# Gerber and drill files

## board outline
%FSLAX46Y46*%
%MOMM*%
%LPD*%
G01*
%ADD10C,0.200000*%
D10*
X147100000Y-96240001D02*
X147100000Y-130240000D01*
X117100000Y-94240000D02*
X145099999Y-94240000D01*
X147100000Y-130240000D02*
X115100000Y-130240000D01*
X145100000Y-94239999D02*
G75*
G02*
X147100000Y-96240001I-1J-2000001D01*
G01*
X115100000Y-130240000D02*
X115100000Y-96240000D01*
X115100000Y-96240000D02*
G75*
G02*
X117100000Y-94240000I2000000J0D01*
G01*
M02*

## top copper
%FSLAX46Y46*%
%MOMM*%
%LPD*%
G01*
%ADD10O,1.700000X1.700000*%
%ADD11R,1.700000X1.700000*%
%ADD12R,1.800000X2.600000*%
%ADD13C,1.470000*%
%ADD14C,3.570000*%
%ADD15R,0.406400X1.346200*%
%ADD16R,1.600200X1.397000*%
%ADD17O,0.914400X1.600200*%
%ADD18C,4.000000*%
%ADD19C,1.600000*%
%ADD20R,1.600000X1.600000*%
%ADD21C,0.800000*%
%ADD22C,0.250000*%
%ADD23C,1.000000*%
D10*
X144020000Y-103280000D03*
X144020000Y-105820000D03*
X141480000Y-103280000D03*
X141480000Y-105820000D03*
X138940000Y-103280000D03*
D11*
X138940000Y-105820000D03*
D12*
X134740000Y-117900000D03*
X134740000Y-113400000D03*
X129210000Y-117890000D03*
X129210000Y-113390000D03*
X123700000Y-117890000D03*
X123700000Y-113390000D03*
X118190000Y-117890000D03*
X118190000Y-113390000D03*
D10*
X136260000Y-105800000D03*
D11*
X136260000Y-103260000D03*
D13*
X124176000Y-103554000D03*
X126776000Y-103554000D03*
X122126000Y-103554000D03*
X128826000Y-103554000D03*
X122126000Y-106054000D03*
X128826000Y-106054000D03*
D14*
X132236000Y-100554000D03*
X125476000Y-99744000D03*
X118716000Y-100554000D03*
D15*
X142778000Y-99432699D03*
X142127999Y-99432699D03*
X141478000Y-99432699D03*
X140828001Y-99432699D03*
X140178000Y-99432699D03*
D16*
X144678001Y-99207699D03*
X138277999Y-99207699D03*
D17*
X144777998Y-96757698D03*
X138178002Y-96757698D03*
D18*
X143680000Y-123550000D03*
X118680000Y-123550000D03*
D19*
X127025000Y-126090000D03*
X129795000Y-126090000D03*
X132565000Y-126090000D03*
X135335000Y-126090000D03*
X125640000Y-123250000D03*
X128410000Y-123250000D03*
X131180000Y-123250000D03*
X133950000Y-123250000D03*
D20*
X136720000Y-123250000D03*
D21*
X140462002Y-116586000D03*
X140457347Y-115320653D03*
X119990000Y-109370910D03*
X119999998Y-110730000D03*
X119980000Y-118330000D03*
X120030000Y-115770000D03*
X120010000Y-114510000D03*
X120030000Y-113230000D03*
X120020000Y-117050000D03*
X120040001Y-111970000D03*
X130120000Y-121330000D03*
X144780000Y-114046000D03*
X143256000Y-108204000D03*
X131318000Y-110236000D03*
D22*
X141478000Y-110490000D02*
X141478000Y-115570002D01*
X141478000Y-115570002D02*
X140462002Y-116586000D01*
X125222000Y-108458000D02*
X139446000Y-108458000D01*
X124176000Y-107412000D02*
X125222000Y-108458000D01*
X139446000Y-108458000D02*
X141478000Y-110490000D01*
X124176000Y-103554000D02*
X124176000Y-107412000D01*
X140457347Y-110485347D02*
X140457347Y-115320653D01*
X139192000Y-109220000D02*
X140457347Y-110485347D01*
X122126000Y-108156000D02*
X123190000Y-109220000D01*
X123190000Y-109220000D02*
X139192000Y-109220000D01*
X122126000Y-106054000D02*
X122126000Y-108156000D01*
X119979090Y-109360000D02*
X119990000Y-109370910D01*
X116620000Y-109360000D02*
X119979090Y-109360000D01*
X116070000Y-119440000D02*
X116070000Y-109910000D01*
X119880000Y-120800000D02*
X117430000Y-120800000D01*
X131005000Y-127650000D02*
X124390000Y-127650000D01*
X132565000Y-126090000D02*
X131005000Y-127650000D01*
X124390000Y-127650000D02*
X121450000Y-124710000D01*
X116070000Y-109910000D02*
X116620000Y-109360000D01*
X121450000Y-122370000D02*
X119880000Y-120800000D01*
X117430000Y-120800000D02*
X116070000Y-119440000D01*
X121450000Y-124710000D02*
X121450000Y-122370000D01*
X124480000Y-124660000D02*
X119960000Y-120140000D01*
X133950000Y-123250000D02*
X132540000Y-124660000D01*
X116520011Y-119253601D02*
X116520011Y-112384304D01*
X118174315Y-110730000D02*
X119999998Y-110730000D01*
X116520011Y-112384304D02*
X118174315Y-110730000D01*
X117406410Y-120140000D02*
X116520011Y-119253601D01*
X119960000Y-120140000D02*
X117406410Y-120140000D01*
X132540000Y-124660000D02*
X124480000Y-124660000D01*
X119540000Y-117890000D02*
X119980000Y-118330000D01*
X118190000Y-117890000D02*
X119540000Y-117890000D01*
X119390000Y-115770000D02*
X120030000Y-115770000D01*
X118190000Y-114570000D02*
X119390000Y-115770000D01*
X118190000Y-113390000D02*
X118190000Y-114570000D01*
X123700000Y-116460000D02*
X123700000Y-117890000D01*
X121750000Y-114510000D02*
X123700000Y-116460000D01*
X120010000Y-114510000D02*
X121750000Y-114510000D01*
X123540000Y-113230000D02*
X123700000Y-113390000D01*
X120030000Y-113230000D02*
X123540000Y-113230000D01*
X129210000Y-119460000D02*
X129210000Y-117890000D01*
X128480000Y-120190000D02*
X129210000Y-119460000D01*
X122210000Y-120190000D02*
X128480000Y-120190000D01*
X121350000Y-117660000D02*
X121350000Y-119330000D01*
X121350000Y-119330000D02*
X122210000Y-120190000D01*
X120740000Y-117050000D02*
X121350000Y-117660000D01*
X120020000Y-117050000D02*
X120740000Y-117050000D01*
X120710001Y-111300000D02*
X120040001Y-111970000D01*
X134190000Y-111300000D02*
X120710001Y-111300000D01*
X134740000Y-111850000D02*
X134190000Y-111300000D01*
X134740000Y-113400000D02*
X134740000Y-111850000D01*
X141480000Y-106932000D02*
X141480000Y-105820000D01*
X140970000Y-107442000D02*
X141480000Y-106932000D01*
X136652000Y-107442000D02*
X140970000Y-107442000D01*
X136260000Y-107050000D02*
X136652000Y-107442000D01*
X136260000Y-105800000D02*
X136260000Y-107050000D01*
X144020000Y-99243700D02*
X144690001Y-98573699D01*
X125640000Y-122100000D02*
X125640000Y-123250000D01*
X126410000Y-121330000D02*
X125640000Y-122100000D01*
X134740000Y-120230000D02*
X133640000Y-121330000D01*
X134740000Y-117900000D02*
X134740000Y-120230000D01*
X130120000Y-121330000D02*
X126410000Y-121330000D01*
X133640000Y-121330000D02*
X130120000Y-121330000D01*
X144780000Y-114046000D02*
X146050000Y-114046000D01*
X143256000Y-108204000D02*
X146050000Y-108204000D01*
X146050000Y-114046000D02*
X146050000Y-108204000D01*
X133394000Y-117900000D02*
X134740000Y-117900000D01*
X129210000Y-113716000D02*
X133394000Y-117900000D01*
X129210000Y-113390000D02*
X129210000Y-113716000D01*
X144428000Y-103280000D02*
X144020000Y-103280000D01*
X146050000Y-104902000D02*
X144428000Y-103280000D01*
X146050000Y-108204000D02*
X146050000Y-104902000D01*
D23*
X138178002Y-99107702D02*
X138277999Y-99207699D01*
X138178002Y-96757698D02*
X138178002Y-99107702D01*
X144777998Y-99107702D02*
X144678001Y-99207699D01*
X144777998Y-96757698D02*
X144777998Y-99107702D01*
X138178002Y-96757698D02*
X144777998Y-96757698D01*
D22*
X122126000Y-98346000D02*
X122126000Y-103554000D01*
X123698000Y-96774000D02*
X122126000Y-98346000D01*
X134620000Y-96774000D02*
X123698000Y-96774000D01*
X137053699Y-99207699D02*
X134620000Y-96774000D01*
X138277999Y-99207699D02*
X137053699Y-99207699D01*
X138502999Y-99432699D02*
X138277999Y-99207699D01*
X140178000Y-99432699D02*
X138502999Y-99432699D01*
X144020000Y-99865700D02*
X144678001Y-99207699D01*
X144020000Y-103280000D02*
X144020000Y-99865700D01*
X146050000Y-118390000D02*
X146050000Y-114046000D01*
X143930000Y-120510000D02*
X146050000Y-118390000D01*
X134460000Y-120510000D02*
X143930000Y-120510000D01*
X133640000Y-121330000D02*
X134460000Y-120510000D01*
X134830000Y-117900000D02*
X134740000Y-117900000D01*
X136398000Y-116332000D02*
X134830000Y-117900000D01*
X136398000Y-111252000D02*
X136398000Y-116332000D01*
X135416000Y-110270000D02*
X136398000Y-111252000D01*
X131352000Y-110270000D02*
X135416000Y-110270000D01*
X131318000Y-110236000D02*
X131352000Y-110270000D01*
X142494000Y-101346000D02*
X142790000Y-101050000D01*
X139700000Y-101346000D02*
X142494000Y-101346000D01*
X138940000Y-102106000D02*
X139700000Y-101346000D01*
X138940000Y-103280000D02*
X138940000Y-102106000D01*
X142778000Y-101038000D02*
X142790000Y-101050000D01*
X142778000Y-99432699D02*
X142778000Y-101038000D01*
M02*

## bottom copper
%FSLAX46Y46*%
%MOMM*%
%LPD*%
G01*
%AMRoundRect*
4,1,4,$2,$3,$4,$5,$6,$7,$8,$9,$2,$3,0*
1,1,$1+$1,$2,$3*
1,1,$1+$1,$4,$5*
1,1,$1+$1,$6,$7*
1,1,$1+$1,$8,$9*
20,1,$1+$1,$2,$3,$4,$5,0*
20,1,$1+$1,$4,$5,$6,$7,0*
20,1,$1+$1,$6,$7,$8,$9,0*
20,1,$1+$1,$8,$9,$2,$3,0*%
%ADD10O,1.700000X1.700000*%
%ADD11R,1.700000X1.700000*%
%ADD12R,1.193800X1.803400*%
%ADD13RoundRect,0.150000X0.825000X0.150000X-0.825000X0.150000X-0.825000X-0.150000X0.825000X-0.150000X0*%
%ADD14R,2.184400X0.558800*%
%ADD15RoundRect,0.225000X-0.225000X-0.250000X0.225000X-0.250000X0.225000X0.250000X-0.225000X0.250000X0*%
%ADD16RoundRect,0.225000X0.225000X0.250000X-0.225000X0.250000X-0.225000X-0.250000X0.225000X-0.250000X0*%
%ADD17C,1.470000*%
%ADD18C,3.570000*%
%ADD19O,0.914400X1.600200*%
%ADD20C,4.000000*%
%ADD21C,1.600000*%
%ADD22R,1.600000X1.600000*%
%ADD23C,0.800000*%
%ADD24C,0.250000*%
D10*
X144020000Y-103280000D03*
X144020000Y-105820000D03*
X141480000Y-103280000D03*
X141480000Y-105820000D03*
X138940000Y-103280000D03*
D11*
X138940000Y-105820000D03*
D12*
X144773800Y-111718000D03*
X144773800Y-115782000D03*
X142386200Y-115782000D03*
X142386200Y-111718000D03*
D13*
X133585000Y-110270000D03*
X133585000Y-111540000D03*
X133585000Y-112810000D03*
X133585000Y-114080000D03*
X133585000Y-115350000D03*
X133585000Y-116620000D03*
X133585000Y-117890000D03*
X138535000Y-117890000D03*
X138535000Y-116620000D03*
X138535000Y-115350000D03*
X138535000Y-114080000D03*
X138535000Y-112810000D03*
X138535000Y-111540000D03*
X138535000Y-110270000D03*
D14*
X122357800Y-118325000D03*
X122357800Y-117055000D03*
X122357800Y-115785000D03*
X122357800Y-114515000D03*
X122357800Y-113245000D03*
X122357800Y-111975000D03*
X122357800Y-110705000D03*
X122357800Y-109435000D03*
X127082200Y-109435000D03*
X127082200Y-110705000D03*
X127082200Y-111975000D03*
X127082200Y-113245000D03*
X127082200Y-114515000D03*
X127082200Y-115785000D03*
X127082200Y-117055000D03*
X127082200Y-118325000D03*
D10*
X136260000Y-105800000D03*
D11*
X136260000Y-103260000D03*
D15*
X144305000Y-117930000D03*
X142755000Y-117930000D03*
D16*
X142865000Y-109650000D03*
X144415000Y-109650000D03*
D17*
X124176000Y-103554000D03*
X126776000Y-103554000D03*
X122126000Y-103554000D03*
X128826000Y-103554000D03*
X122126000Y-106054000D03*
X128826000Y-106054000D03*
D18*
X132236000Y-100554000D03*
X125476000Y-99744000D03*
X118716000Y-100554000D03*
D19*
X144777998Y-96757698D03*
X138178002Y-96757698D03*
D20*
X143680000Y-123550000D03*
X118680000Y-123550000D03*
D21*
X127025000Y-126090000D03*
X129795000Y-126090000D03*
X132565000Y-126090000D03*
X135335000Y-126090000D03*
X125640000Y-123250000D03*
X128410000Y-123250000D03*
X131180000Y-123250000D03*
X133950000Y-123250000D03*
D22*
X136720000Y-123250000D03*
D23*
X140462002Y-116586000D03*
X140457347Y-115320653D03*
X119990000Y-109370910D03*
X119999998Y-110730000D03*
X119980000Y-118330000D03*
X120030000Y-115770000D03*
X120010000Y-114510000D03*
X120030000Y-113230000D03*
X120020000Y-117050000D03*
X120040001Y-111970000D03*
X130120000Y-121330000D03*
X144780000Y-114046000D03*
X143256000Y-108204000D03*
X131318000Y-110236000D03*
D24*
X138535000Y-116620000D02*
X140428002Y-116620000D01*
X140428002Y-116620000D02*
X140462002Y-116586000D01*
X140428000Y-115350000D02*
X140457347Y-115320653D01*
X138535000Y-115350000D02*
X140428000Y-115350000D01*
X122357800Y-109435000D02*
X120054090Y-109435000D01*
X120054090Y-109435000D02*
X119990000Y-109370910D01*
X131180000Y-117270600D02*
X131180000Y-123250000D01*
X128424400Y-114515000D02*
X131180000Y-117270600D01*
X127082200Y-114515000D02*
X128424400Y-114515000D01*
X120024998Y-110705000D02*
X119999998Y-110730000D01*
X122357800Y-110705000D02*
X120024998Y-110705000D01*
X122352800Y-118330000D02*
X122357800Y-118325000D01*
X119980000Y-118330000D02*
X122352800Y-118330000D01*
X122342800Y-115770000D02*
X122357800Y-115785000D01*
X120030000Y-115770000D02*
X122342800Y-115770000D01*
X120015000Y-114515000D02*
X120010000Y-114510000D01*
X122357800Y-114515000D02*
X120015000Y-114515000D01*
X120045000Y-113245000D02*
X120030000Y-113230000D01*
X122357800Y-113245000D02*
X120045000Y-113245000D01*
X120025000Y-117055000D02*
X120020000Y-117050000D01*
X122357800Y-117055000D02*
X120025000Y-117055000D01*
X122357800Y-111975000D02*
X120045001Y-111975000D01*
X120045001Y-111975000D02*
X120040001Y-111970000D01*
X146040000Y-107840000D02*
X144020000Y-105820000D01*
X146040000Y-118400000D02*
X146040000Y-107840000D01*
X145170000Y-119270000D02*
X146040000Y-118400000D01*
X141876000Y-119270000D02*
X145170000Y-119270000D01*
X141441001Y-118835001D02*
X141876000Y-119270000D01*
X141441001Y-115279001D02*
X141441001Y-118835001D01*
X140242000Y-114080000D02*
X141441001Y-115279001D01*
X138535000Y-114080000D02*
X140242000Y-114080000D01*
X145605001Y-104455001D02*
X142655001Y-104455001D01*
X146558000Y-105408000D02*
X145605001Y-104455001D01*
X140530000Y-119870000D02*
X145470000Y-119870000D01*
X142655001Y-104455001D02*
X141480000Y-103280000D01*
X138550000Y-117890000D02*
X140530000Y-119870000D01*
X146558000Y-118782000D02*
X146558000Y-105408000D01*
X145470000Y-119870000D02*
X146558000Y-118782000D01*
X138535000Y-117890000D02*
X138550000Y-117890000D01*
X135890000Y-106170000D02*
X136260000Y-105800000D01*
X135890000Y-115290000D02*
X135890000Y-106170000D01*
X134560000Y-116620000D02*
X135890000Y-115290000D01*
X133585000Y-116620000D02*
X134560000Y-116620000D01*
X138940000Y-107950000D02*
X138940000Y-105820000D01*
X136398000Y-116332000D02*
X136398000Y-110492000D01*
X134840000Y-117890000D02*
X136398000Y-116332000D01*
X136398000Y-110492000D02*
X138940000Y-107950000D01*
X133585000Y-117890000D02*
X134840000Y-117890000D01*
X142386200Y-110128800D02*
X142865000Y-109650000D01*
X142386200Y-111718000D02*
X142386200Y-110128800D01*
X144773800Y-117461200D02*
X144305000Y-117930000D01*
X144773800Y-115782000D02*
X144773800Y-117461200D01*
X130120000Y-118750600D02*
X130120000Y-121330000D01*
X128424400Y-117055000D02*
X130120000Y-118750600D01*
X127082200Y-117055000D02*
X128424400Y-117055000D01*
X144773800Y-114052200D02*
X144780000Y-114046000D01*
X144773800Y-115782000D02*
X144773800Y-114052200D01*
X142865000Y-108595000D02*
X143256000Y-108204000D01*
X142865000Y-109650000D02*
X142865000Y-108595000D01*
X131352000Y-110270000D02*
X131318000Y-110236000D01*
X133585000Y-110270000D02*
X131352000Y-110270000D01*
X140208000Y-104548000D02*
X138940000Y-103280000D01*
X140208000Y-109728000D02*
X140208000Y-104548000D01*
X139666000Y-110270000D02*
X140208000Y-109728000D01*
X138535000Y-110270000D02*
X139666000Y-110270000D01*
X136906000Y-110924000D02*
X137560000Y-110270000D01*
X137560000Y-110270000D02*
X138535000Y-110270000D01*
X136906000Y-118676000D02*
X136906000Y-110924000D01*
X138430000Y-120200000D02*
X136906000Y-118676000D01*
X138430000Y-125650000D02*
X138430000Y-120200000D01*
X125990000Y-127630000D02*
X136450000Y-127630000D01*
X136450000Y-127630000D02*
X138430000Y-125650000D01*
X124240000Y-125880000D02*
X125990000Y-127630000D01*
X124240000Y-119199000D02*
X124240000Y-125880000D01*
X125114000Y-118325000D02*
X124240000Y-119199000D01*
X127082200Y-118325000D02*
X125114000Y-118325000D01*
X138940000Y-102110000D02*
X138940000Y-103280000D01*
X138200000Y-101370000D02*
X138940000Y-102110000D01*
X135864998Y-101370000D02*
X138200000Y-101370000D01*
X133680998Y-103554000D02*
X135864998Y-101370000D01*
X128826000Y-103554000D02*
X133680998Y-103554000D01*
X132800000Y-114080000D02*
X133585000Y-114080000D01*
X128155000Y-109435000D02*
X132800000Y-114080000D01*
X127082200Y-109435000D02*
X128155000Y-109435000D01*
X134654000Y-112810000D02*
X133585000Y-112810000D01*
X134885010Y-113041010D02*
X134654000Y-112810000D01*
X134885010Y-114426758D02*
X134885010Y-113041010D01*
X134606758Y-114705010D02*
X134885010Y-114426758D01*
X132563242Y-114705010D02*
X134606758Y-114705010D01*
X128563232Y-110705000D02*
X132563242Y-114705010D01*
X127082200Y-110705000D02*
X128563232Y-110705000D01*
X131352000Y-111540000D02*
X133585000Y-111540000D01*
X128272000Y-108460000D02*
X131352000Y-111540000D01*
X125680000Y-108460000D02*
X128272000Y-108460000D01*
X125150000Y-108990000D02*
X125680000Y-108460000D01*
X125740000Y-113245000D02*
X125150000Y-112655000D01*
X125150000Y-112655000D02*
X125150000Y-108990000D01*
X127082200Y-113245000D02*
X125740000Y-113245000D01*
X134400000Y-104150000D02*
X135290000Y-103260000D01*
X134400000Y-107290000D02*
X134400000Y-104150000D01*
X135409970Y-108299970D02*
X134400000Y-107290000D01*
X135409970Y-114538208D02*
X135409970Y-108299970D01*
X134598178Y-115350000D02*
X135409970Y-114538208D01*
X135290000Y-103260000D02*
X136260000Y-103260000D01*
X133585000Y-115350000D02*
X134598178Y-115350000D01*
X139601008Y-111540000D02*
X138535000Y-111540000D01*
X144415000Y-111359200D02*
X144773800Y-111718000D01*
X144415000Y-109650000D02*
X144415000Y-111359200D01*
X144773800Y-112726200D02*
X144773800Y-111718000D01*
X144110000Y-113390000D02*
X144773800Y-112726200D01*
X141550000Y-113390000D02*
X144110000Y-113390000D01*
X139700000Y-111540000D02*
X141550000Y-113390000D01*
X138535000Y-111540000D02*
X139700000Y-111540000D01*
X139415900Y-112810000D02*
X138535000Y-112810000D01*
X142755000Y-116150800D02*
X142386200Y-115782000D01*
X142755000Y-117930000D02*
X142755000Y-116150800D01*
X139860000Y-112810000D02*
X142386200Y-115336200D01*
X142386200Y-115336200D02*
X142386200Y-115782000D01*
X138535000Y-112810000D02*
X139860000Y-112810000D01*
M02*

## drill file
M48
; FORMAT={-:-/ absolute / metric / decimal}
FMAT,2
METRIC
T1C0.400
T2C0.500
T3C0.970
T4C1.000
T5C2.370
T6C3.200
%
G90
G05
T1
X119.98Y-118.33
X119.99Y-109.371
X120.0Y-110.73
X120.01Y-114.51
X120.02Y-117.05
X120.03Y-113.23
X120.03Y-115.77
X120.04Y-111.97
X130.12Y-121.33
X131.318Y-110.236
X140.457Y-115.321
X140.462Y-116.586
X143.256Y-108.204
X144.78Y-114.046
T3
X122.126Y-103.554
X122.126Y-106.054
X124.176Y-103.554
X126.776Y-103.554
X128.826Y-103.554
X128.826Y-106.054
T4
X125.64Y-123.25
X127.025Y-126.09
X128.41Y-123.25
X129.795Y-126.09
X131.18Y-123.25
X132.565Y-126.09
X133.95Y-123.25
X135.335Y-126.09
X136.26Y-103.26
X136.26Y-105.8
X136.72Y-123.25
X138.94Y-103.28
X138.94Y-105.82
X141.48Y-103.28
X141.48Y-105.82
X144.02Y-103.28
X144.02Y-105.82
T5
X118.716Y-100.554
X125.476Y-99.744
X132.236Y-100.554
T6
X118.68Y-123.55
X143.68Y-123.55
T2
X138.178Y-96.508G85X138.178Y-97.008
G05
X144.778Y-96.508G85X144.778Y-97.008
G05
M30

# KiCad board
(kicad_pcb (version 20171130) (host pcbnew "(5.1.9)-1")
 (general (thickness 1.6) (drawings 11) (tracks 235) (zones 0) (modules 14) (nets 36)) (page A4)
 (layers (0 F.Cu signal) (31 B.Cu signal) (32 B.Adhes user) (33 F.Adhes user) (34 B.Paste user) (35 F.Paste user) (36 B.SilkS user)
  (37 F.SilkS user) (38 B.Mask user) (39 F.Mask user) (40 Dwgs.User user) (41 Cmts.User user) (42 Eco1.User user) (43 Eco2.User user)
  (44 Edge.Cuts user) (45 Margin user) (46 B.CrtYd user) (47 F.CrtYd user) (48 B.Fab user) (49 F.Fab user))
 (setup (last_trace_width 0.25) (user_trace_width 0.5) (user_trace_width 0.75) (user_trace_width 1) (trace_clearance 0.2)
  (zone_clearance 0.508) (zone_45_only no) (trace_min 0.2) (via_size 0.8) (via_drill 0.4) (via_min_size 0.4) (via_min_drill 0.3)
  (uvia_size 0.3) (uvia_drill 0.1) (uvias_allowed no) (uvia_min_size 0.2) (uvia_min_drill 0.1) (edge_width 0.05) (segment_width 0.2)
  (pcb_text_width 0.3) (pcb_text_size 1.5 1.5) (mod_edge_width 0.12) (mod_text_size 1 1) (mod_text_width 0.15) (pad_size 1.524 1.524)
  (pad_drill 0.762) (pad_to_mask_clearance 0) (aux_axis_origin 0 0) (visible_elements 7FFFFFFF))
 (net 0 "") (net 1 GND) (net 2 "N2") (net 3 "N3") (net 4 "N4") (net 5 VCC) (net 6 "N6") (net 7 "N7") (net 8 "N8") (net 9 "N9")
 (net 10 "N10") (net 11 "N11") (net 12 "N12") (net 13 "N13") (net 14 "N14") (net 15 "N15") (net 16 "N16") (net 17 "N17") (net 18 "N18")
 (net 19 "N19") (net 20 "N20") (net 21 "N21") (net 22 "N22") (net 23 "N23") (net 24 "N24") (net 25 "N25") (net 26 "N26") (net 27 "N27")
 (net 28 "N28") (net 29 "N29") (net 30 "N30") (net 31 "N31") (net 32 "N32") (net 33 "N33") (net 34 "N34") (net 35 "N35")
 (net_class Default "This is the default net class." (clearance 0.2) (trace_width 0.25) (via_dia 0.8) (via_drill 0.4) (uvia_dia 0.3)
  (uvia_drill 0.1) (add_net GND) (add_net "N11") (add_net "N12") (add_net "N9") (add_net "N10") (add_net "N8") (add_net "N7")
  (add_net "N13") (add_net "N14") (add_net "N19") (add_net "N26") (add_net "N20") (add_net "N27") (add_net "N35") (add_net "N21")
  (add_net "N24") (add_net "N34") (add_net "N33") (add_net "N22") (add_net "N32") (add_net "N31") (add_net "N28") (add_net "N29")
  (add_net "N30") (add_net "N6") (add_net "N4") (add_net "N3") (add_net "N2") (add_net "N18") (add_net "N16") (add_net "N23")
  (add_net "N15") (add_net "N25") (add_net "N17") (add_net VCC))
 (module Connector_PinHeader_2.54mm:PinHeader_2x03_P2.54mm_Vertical (layer F.Cu) (at 138.94 105.82 90)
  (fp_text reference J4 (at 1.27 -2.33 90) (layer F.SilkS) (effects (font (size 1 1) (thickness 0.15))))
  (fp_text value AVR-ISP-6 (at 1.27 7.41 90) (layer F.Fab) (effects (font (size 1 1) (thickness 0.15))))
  (pad 6 thru_hole oval (at 2.54 5.08 90) (size 1.7 1.7) (drill 1) (layers *.Cu *.Mask) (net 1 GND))
  (pad 5 thru_hole oval (at 0 5.08 90) (size 1.7 1.7) (drill 1) (layers *.Cu *.Mask) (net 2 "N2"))
  (pad 4 thru_hole oval (at 2.54 2.54 90) (size 1.7 1.7) (drill 1) (layers *.Cu *.Mask) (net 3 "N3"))
  (pad 3 thru_hole oval (at 0 2.54 90) (size 1.7 1.7) (drill 1) (layers *.Cu *.Mask) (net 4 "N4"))
  (pad 2 thru_hole oval (at 2.54 0 90) (size 1.7 1.7) (drill 1) (layers *.Cu *.Mask) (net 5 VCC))
  (pad 1 thru_hole rect (at 0 0 90) (size 1.7 1.7) (drill 1) (layers *.Cu *.Mask) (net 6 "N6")))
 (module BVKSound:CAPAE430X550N (layer F.Cu) (at 134.74 115.65 90)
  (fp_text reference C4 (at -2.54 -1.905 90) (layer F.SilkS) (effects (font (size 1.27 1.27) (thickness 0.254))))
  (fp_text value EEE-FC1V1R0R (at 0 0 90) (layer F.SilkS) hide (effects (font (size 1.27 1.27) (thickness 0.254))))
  (pad 1 smd rect (at -2.25 0 180) (size 1.8 2.6) (layers F.Cu F.Paste F.Mask) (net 1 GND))
  (pad 2 smd rect (at 2.25 0 180) (size 1.8 2.6) (layers F.Cu F.Paste F.Mask) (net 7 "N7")))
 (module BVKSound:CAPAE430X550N (layer F.Cu) (at 129.21 115.64 90)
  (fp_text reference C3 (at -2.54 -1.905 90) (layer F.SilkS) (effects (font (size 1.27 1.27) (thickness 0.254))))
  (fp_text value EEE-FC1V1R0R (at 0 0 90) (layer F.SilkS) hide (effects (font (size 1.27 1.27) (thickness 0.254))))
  (pad 1 smd rect (at -2.25 0 180) (size 1.8 2.6) (layers F.Cu F.Paste F.Mask) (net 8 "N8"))
  (pad 2 smd rect (at 2.25 0 180) (size 1.8 2.6) (layers F.Cu F.Paste F.Mask) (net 1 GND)))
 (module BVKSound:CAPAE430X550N (layer F.Cu) (at 123.7 115.64 90)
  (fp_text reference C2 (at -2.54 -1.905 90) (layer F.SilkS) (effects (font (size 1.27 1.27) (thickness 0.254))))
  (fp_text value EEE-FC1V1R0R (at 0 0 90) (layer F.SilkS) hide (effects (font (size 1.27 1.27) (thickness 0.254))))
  (pad 1 smd rect (at -2.25 0 180) (size 1.8 2.6) (layers F.Cu F.Paste F.Mask) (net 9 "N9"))
  (pad 2 smd rect (at 2.25 0 180) (size 1.8 2.6) (layers F.Cu F.Paste F.Mask) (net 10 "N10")))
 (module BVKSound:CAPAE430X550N (layer F.Cu) (at 118.19 115.64 90)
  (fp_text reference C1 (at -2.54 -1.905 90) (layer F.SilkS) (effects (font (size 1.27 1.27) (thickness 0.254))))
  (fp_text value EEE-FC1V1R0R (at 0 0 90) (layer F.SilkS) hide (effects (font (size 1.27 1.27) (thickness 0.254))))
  (pad 1 smd rect (at -2.25 0 180) (size 1.8 2.6) (layers F.Cu F.Paste F.Mask) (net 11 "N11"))
  (pad 2 smd rect (at 2.25 0 180) (size 1.8 2.6) (layers F.Cu F.Paste F.Mask) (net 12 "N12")))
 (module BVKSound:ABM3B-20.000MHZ (layer B.Cu) (at 143.58 113.75 180)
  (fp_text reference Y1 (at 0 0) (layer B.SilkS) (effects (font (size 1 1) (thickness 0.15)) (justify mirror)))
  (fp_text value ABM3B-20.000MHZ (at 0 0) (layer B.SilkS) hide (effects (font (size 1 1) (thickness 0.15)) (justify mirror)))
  (pad 1 smd rect (at -1.1938 2.032 180) (size 1.1938 1.8034) (layers B.Cu B.Paste B.Mask) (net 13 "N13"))
  (pad 2 smd rect (at -1.1938 -2.032 180) (size 1.1938 1.8034) (layers B.Cu B.Paste B.Mask) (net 1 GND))
  (pad 3 smd rect (at 1.1938 -2.032 180) (size 1.1938 1.8034) (layers B.Cu B.Paste B.Mask) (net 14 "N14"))
  (pad 4 smd rect (at 1.1938 2.032 180) (size 1.1938 1.8034) (layers B.Cu B.Paste B.Mask) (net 1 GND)))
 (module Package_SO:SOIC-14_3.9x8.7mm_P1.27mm (layer B.Cu) (at 136.06 114.08 180)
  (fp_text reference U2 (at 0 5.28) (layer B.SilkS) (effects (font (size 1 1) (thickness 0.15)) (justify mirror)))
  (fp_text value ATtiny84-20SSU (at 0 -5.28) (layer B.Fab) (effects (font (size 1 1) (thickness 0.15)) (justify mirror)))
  (pad 14 smd roundrect (at 2.475 3.81 180) (size 1.95 0.6) (layers B.Cu B.Paste B.Mask) (roundrect_rratio 0.25) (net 1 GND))
  (pad 13 smd roundrect (at 2.475 2.54 180) (size 1.95 0.6) (layers B.Cu B.Paste B.Mask) (roundrect_rratio 0.25) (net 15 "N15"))
  (pad 12 smd roundrect (at 2.475 1.27 180) (size 1.95 0.6) (layers B.Cu B.Paste B.Mask) (roundrect_rratio 0.25) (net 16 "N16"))
  (pad 11 smd roundrect (at 2.475 0 180) (size 1.95 0.6) (layers B.Cu B.Paste B.Mask) (roundrect_rratio 0.25) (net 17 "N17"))
  (pad 10 smd roundrect (at 2.475 -1.27 180) (size 1.95 0.6) (layers B.Cu B.Paste B.Mask) (roundrect_rratio 0.25) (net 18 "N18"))
  (pad 9 smd roundrect (at 2.475 -2.54 180) (size 1.95 0.6) (layers B.Cu B.Paste B.Mask) (roundrect_rratio 0.25) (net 4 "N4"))
  (pad 8 smd roundrect (at 2.475 -3.81 180) (size 1.95 0.6) (layers B.Cu B.Paste B.Mask) (roundrect_rratio 0.25) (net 6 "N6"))
  (pad 7 smd roundrect (at -2.475 -3.81 180) (size 1.95 0.6) (layers B.Cu B.Paste B.Mask) (roundrect_rratio 0.25) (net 3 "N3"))
  (pad 6 smd roundrect (at -2.475 -2.54 180) (size 1.95 0.6) (layers B.Cu B.Paste B.Mask) (roundrect_rratio 0.25) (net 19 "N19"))
  (pad 5 smd roundrect (at -2.475 -1.27 180) (size 1.95 0.6) (layers B.Cu B.Paste B.Mask) (roundrect_rratio 0.25) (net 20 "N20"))
  (pad 4 smd roundrect (at -2.475 0 180) (size 1.95 0.6) (layers B.Cu B.Paste B.Mask) (roundrect_rratio 0.25) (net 2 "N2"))
  (pad 3 smd roundrect (at -2.475 1.27 180) (size 1.95 0.6) (layers B.Cu B.Paste B.Mask) (roundrect_rratio 0.25) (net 14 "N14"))
  (pad 2 smd roundrect (at -2.475 2.54 180) (size 1.95 0.6) (layers B.Cu B.Paste B.Mask) (roundrect_rratio 0.25) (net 13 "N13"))
  (pad 1 smd roundrect (at -2.475 3.81 180) (size 1.95 0.6) (layers B.Cu B.Paste B.Mask) (roundrect_rratio 0.25) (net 5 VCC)))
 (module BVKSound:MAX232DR (layer B.Cu) (at 124.72 113.88)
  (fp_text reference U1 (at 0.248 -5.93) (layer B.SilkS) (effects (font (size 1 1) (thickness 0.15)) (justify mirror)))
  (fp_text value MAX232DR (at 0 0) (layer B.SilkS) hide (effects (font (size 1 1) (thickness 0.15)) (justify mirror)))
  (pad 1 smd rect (at -2.3622 4.445) (size 2.1844 0.5588) (layers B.Cu B.Paste B.Mask) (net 11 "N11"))
  (pad 2 smd rect (at -2.3622 3.175) (size 2.1844 0.5588) (layers B.Cu B.Paste B.Mask) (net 8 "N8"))
  (pad 3 smd rect (at -2.3622 1.905) (size 2.1844 0.5588) (layers B.Cu B.Paste B.Mask) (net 12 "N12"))
  (pad 4 smd rect (at -2.3622 0.635) (size 2.1844 0.5588) (layers B.Cu B.Paste B.Mask) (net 9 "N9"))
  (pad 5 smd rect (at -2.3622 -0.635) (size 2.1844 0.5588) (layers B.Cu B.Paste B.Mask) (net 10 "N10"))
  (pad 6 smd rect (at -2.3622 -1.905) (size 2.1844 0.5588) (layers B.Cu B.Paste B.Mask) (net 7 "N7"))
  (pad 7 smd rect (at -2.3622 -3.175) (size 2.1844 0.5588) (layers B.Cu B.Paste B.Mask) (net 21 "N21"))
  (pad 8 smd rect (at -2.3622 -4.445) (size 2.1844 0.5588) (layers B.Cu B.Paste B.Mask) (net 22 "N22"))
  (pad 9 smd rect (at 2.3622 -4.445) (size 2.1844 0.5588) (layers B.Cu B.Paste B.Mask) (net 17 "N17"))
  (pad 10 smd rect (at 2.3622 -3.175) (size 2.1844 0.5588) (layers B.Cu B.Paste B.Mask) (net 16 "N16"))
  (pad 11 smd rect (at 2.3622 -1.905) (size 2.1844 0.5588) (layers B.Cu B.Paste B.Mask) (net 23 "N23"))
  (pad 12 smd rect (at 2.3622 -0.635) (size 2.1844 0.5588) (layers B.Cu B.Paste B.Mask) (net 15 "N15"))
  (pad 13 smd rect (at 2.3622 0.635) (size 2.1844 0.5588) (layers B.Cu B.Paste B.Mask) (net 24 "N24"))
  (pad 14 smd rect (at 2.3622 1.905) (size 2.1844 0.5588) (layers B.Cu B.Paste B.Mask) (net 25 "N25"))
  (pad 15 smd rect (at 2.3622 3.175) (size 2.1844 0.5588) (layers B.Cu B.Paste B.Mask) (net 1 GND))
  (pad 16 smd rect (at 2.3622 4.445) (size 2.1844 0.5588) (layers B.Cu B.Paste B.Mask) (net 5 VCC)))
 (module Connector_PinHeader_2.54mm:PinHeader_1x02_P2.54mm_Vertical (layer F.Cu) (at 136.26 103.26)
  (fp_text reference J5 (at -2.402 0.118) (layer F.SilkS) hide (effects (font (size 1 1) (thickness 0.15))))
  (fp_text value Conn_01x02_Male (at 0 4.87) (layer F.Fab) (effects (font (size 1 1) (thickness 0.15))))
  (pad 2 thru_hole oval (at 0 2.54) (size 1.7 1.7) (drill 1) (layers *.Cu *.Mask) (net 4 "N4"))
  (pad 1 thru_hole rect (at 0 0) (size 1.7 1.7) (drill 1) (layers *.Cu *.Mask) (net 18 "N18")))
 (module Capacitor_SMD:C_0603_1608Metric (layer B.Cu) (at 143.53 117.93)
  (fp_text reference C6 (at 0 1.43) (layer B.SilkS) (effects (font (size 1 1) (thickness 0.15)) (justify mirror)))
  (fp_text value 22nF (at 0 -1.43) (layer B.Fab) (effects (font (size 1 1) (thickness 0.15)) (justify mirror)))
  (pad 2 smd roundrect (at 0.775 0) (size 0.9 0.95) (layers B.Cu B.Paste B.Mask) (roundrect_rratio 0.25) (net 1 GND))
  (pad 1 smd roundrect (at -0.775 0) (size 0.9 0.95) (layers B.Cu B.Paste B.Mask) (roundrect_rratio 0.25) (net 14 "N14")))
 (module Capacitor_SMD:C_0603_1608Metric (layer B.Cu) (at 143.64 109.65 180)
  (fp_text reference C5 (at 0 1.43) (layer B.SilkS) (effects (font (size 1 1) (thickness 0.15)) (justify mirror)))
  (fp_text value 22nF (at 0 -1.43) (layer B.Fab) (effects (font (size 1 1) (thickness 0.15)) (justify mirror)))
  (pad 2 smd roundrect (at 0.775 0 180) (size 0.9 0.95) (layers B.Cu B.Paste B.Mask) (roundrect_rratio 0.25) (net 1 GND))
  (pad 1 smd roundrect (at -0.775 0 180) (size 0.9 0.95) (layers B.Cu B.Paste B.Mask) (roundrect_rratio 0.25) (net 13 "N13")))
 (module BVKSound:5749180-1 (layer B.Cu) (at 125.476 94.234 180)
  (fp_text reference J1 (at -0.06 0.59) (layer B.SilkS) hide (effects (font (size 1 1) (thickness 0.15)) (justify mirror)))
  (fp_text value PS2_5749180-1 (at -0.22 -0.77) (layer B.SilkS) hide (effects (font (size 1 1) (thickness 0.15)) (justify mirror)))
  (pad 1 thru_hole circle (at 1.3 -9.32 180) (size 1.47 1.47) (drill 0.97) (layers *.Cu *.Mask) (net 19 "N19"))
  (pad 2 thru_hole circle (at -1.3 -9.32 180) (size 1.47 1.47) (drill 0.97) (layers *.Cu *.Mask) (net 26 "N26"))
  (pad 3 thru_hole circle (at 3.35 -9.32 180) (size 1.47 1.47) (drill 0.97) (layers *.Cu *.Mask) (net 1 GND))
  (pad 4 thru_hole circle (at -3.35 -9.32 180) (size 1.47 1.47) (drill 0.97) (layers *.Cu *.Mask) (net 5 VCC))
  (pad 5 thru_hole circle (at 3.35 -11.82 180) (size 1.47 1.47) (drill 0.97) (layers *.Cu *.Mask) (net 20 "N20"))
  (pad 6 thru_hole circle (at -3.35 -11.82 180) (size 1.47 1.47) (drill 0.97) (layers *.Cu *.Mask) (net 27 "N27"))
  (pad 7 thru_hole circle (at -6.76 -6.32 180) (size 3.57 3.57) (drill 2.37) (layers *.Cu *.Mask))
  (pad 8 thru_hole circle (at 0 -5.51 180) (size 3.57 3.57) (drill 2.37) (layers *.Cu *.Mask))
  (pad 9 thru_hole circle (at 6.76 -6.32 180) (size 3.57 3.57) (drill 2.37) (layers *.Cu *.Mask)))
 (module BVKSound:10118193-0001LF (layer F.Cu) (at 141.478 96.774 180)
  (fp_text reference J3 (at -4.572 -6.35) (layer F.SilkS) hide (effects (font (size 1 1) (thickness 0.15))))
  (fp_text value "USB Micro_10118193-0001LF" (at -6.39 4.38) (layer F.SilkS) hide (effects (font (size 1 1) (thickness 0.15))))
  (pad 1 smd rect (at -1.3 -2.658699 180) (size 0.4064 1.3462) (layers F.Cu F.Paste F.Mask) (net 5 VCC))
  (pad 2 smd rect (at -0.649999 -2.658699 180) (size 0.4064 1.3462) (layers F.Cu F.Paste F.Mask) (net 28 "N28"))
  (pad 3 smd rect (at 0 -2.658699 180) (size 0.4064 1.3462) (layers F.Cu F.Paste F.Mask) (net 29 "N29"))
  (pad 4 smd rect (at 0.649999 -2.658699 180) (size 0.4064 1.3462) (layers F.Cu F.Paste F.Mask) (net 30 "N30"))
  (pad 5 smd rect (at 1.3 -2.658699 180) (size 0.4064 1.3462) (layers F.Cu F.Paste F.Mask) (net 1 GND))
  (pad 5 smd rect (at -3.200001 -2.433699 180) (size 1.6002 1.397) (layers F.Cu F.Paste F.Mask) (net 1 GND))
  (pad 5 smd rect (at 3.200001 -2.433699 180) (size 1.6002 1.397) (layers F.Cu F.Paste F.Mask) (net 1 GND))
  (pad 5 thru_hole oval (at -3.299998 0.016302 270) (size 1.6002 0.9144) (drill oval 1 0.5) (layers *.Cu *.Mask) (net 1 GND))
  (pad 5 thru_hole oval (at 3.299998 0.016302 270) (size 1.6002 0.9144) (drill oval 1 0.5) (layers *.Cu *.Mask) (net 1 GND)))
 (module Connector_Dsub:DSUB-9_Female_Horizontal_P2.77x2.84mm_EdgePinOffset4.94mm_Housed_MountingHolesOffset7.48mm (layer F.Cu)
  (at 136.72 123.25)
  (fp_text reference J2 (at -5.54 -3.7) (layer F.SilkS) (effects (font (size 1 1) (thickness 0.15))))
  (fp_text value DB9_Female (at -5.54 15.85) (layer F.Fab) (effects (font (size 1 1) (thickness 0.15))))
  (pad 0 thru_hole circle (at 6.96 0.3) (size 4 4) (drill 3.2) (layers *.Cu *.Mask))
  (pad 0 thru_hole circle (at -18.04 0.3) (size 4 4) (drill 3.2) (layers *.Cu *.Mask))
  (pad 9 thru_hole circle (at -9.695 2.84) (size 1.6 1.6) (drill 1) (layers *.Cu *.Mask) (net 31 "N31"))
  (pad 8 thru_hole circle (at -6.925 2.84) (size 1.6 1.6) (drill 1) (layers *.Cu *.Mask) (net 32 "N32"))
  (pad 7 thru_hole circle (at -4.155 2.84) (size 1.6 1.6) (drill 1) (layers *.Cu *.Mask) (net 22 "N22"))
  (pad 6 thru_hole circle (at -1.385 2.84) (size 1.6 1.6) (drill 1) (layers *.Cu *.Mask) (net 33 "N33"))
  (pad 5 thru_hole circle (at -11.08 0) (size 1.6 1.6) (drill 1) (layers *.Cu *.Mask) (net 1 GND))
  (pad 4 thru_hole circle (at -8.31 0) (size 1.6 1.6) (drill 1) (layers *.Cu *.Mask) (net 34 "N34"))
  (pad 3 thru_hole circle (at -5.54 0) (size 1.6 1.6) (drill 1) (layers *.Cu *.Mask) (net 24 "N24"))
  (pad 2 thru_hole circle (at -2.77 0) (size 1.6 1.6) (drill 1) (layers *.Cu *.Mask) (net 21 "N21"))
  (pad 1 thru_hole rect (at 0 0) (size 1.6 1.6) (drill 1) (layers *.Cu *.Mask) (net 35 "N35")))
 (gr_line (start 147.1 96.240001) (end 147.1 130.24) (layer Edge.Cuts) (width 0.2))
 (gr_line (start 117.1 94.24) (end 145.099999 94.24) (layer Edge.Cuts) (width 0.2))
 (gr_line (start 147.1 130.24) (end 115.1 130.24) (layer Edge.Cuts) (width 0.2))
 (gr_arc (start 145.099999 96.24) (end 147.1 96.240001) (angle -90) (layer Edge.Cuts) (width 0.2))
 (gr_line (start 115.1 130.24) (end 115.1 96.24) (layer Edge.Cuts) (width 0.2))
 (gr_arc (start 117.1 96.24) (end 117.1 94.24) (angle -90) (layer Edge.Cuts) (width 0.2))
 (segment (start 138.535 116.62) (end 140.428002 116.62) (width 0.25) (layer B.Cu) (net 19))
 (via (at 140.462002 116.586) (size 0.8) (drill 0.4) (layers F.Cu B.Cu) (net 19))
 (segment (start 140.428002 116.62) (end 140.462002 116.586) (width 0.25) (layer B.Cu) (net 19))
 (segment (start 141.478 110.49) (end 141.478 115.570002) (width 0.25) (layer F.Cu) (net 19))
 (segment (start 141.478 115.570002) (end 140.462002 116.586) (width 0.25) (layer F.Cu) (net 19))
 (segment (start 125.222 108.458) (end 139.446 108.458) (width 0.25) (layer F.Cu) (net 19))
 (segment (start 124.176 107.412) (end 125.222 108.458) (width 0.25) (layer F.Cu) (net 19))
 (segment (start 139.446 108.458) (end 141.478 110.49) (width 0.25) (layer F.Cu) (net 19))
 (segment (start 124.176 103.554) (end 124.176 107.412) (width 0.25) (layer F.Cu) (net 19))
 (via (at 140.457347 115.320653) (size 0.8) (drill 0.4) (layers F.Cu B.Cu) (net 20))
 (segment (start 140.428 115.35) (end 140.457347 115.320653) (width 0.25) (layer B.Cu) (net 20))
 (segment (start 138.535 115.35) (end 140.428 115.35) (width 0.25) (layer B.Cu) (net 20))
 (segment (start 140.457347 110.485347) (end 140.457347 115.320653) (width 0.25) (layer F.Cu) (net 20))
 (segment (start 139.192 109.22) (end 140.457347 110.485347) (width 0.25) (layer F.Cu) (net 20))
 (segment (start 122.126 108.156) (end 123.19 109.22) (width 0.25) (layer F.Cu) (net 20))
 (segment (start 123.19 109.22) (end 139.192 109.22) (width 0.25) (layer F.Cu) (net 20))
 (segment (start 122.126 106.054) (end 122.126 108.156) (width 0.25) (layer F.Cu) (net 20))
 (segment (start 122.3578 109.435) (end 120.05409 109.435) (width 0.25) (layer B.Cu) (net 22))
 (segment (start 120.05409 109.435) (end 119.99 109.37091) (width 0.25) (layer B.Cu) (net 22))
 (via (at 119.99 109.37091) (size 0.8) (drill 0.4) (layers F.Cu B.Cu) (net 22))
 (segment (start 119.97909 109.36) (end 119.99 109.37091) (width 0.25) (layer F.Cu) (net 22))
 (segment (start 116.62 109.36) (end 119.97909 109.36) (width 0.25) (layer F.Cu) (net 22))
 (segment (start 116.07 119.44) (end 116.07 109.91) (width 0.25) (layer F.Cu) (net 22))
 (segment (start 119.88 120.8) (end 117.43 120.8) (width 0.25) (layer F.Cu) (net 22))
 (segment (start 131.005 127.65) (end 124.39 127.65) (width 0.25) (layer F.Cu) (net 22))
 (segment (start 132.565 126.09) (end 131.005 127.65) (width 0.25) (layer F.Cu) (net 22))
 (segment (start 124.39 127.65) (end 121.45 124.71) (width 0.25) (layer F.Cu) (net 22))
 (segment (start 116.07 109.91) (end 116.62 109.36) (width 0.25) (layer F.Cu) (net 22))
 (segment (start 121.45 122.37) (end 119.88 120.8) (width 0.25) (layer F.Cu) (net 22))
 (segment (start 117.43 120.8) (end 116.07 119.44) (width 0.25) (layer F.Cu) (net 22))
 (segment (start 121.45 124.71) (end 121.45 122.37) (width 0.25) (layer F.Cu) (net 22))
 (segment (start 131.18 117.2706) (end 131.18 123.25) (width 0.25) (layer B.Cu) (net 24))
 (segment (start 128.4244 114.515) (end 131.18 117.2706) (width 0.25) (layer B.Cu) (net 24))
 (segment (start 127.0822 114.515) (end 128.4244 114.515) (width 0.25) (layer B.Cu) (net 24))
 (via (at 119.999998 110.73) (size 0.8) (drill 0.4) (layers F.Cu B.Cu) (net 21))
 (segment (start 120.024998 110.705) (end 119.999998 110.73) (width 0.25) (layer B.Cu) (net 21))
 (segment (start 122.3578 110.705) (end 120.024998 110.705) (width 0.25) (layer B.Cu) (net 21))
 (segment (start 124.48 124.66) (end 119.96 120.14) (width 0.25) (layer F.Cu) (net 21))
 (segment (start 133.95 123.25) (end 132.54 124.66) (width 0.25) (layer F.Cu) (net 21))
 (segment (start 116.520011 119.253601) (end 116.520011 112.384304) (width 0.25) (layer F.Cu) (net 21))
 (segment (start 118.174315 110.73) (end 119.999998 110.73) (width 0.25) (layer F.Cu) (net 21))
 (segment (start 116.520011 112.384304) (end 118.174315 110.73) (width 0.25) (layer F.Cu) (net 21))
 (segment (start 117.40641 120.14) (end 116.520011 119.253601) (width 0.25) (layer F.Cu) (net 21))
 (segment (start 119.96 120.14) (end 117.40641 120.14) (width 0.25) (layer F.Cu) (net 21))
 (segment (start 132.54 124.66) (end 124.48 124.66) (width 0.25) (layer F.Cu) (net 21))
 (via (at 119.98 118.33) (size 0.8) (drill 0.4) (layers F.Cu B.Cu) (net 11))
 (segment (start 119.54 117.89) (end 119.98 118.33) (width 0.25) (layer F.Cu) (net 11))
 (segment (start 118.19 117.89) (end 119.54 117.89) (width 0.25) (layer F.Cu) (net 11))
 (segment (start 122.3528 118.33) (end 122.3578 118.325) (width 0.25) (layer B.Cu) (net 11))
 (segment (start 119.98 118.33) (end 122.3528 118.33) (width 0.25) (layer B.Cu) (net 11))
 (via (at 120.03 115.77) (size 0.8) (drill 0.4) (layers F.Cu B.Cu) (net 12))
 (segment (start 122.3428 115.77) (end 122.3578 115.785) (width 0.25) (layer B.Cu) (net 12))
 (segment (start 120.03 115.77) (end 122.3428 115.77) (width 0.25) (layer B.Cu) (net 12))
 (segment (start 119.39 115.77) (end 120.03 115.77) (width 0.25) (layer F.Cu) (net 12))
 (segment (start 118.19 114.57) (end 119.39 115.77) (width 0.25) (layer F.Cu) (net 12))
 (segment (start 118.19 113.39) (end 118.19 114.57) (width 0.25) (layer F.Cu) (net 12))
 (via (at 120.01 114.51) (size 0.8) (drill 0.4) (layers F.Cu B.Cu) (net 9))
 (segment (start 120.015 114.515) (end 120.01 114.51) (width 0.25) (layer B.Cu) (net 9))
 (segment (start 122.3578 114.515) (end 120.015 114.515) (width 0.25) (layer B.Cu) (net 9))
 (segment (start 123.7 116.46) (end 123.7 117.89) (width 0.25) (layer F.Cu) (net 9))
 (segment (start 121.75 114.51) (end 123.7 116.46) (width 0.25) (layer F.Cu) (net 9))
 (segment (start 120.01 114.51) (end 121.75 114.51) (width 0.25) (layer F.Cu) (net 9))
 (via (at 120.03 113.23) (size 0.8) (drill 0.4) (layers F.Cu B.Cu) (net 10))
 (segment (start 120.045 113.245) (end 120.03 113.23) (width 0.25) (layer B.Cu) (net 10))
 (segment (start 122.3578 113.245) (end 120.045 113.245) (width 0.25) (layer B.Cu) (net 10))
 (segment (start 123.54 113.23) (end 123.7 113.39) (width 0.25) (layer F.Cu) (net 10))
 (segment (start 120.03 113.23) (end 123.54 113.23) (width 0.25) (layer F.Cu) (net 10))
 (via (at 120.02 117.05) (size 0.8) (drill 0.4) (layers F.Cu B.Cu) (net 8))
 (segment (start 120.025 117.055) (end 120.02 117.05) (width 0.25) (layer B.Cu) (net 8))
 (segment (start 122.3578 117.055) (end 120.025 117.055) (width 0.25) (layer B.Cu) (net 8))
 (segment (start 129.21 119.46) (end 129.21 117.89) (width 0.25) (layer F.Cu) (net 8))
 (segment (start 128.48 120.19) (end 129.21 119.46) (width 0.25) (layer F.Cu) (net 8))
 (segment (start 122.21 120.19) (end 128.48 120.19) (width 0.25) (layer F.Cu) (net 8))
 (segment (start 121.35 117.66) (end 121.35 119.33) (width 0.25) (layer F.Cu) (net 8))
 (segment (start 121.35 119.33) (end 122.21 120.19) (width 0.25) (layer F.Cu) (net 8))
 (segment (start 120.74 117.05) (end 121.35 117.66) (width 0.25) (layer F.Cu) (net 8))
 (segment (start 120.02 117.05) (end 120.74 117.05) (width 0.25) (layer F.Cu) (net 8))
 (via (at 120.040001 111.97) (size 0.8) (drill 0.4) (layers F.Cu B.Cu) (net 7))
 (segment (start 122.3578 111.975) (end 120.045001 111.975) (width 0.25) (layer B.Cu) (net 7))
 (segment (start 120.045001 111.975) (end 120.040001 111.97) (width 0.25) (layer B.Cu) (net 7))
 (segment (start 120.710001 111.3) (end 120.040001 111.97) (width 0.25) (layer F.Cu) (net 7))
 (segment (start 134.19 111.3) (end 120.710001 111.3) (width 0.25) (layer F.Cu) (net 7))
 (segment (start 134.74 111.85) (end 134.19 111.3) (width 0.25) (layer F.Cu) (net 7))
 (segment (start 134.74 113.4) (end 134.74 111.85) (width 0.25) (layer F.Cu) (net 7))
 (segment (start 146.04 107.84) (end 144.02 105.82) (width 0.25) (layer B.Cu) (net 2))
 (segment (start 146.04 118.4) (end 146.04 107.84) (width 0.25) (layer B.Cu) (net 2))
 (segment (start 145.17 119.27) (end 146.04 118.4) (width 0.25) (layer B.Cu) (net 2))
 (segment (start 141.876 119.27) (end 145.17 119.27) (width 0.25) (layer B.Cu) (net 2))
 (segment (start 141.441001 118.835001) (end 141.876 119.27) (width 0.25) (layer B.Cu) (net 2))
 (segment (start 141.441001 115.279001) (end 141.441001 118.835001) (width 0.25) (layer B.Cu) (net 2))
 (segment (start 140.242 114.08) (end 141.441001 115.279001) (width 0.25) (layer B.Cu) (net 2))
 (segment (start 138.535 114.08) (end 140.242 114.08) (width 0.25) (layer B.Cu) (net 2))
 (segment (start 145.605001 104.455001) (end 142.655001 104.455001) (width 0.25) (layer B.Cu) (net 3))
 (segment (start 146.558 105.408) (end 145.605001 104.455001) (width 0.25) (layer B.Cu) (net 3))
 (segment (start 140.53 119.87) (end 145.47 119.87) (width 0.25) (layer B.Cu) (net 3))
 (segment (start 142.655001 104.455001) (end 141.48 103.28) (width 0.25) (layer B.Cu) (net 3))
 (segment (start 138.55 117.89) (end 140.53 119.87) (width 0.25) (layer B.Cu) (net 3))
 (segment (start 146.558 118.782) (end 146.558 105.408) (width 0.25) (layer B.Cu) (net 3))
 (segment (start 145.47 119.87) (end 146.558 118.782) (width 0.25) (layer B.Cu) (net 3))
 (segment (start 138.535 117.89) (end 138.55 117.89) (width 0.25) (layer B.Cu) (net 3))
 (segment (start 141.48 106.932) (end 141.48 105.82) (width 0.25) (layer F.Cu) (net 4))
 (segment (start 140.97 107.442) (end 141.48 106.932) (width 0.25) (layer F.Cu) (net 4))
 (segment (start 136.652 107.442) (end 140.97 107.442) (width 0.25) (layer F.Cu) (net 4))
 (segment (start 136.26 107.05) (end 136.652 107.442) (width 0.25) (layer F.Cu) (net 4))
 (segment (start 136.26 105.8) (end 136.26 107.05) (width 0.25) (layer F.Cu) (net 4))
 (segment (start 135.89 106.17) (end 136.26 105.8) (width 0.25) (layer B.Cu) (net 4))
 (segment (start 135.89 115.29) (end 135.89 106.17) (width 0.25) (layer B.Cu) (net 4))
 (segment (start 134.56 116.62) (end 135.89 115.29) (width 0.25) (layer B.Cu) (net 4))
 (segment (start 133.585 116.62) (end 134.56 116.62) (width 0.25) (layer B.Cu) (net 4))
 (segment (start 138.94 107.95) (end 138.94 105.82) (width 0.25) (layer B.Cu) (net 6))
 (segment (start 136.398 116.332) (end 136.398 110.492) (width 0.25) (layer B.Cu) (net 6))
 (segment (start 134.84 117.89) (end 136.398 116.332) (width 0.25) (layer B.Cu) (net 6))
 (segment (start 136.398 110.492) (end 138.94 107.95) (width 0.25) (layer B.Cu) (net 6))
 (segment (start 133.585 117.89) (end 134.84 117.89) (width 0.25) (layer B.Cu) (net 6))
 (segment (start 142.3862 110.1288) (end 142.865 109.65) (width 0.25) (layer B.Cu) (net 1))
 (segment (start 142.3862 111.718) (end 142.3862 110.1288) (width 0.25) (layer B.Cu) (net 1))
 (segment (start 144.7738 117.4612) (end 144.305 117.93) (width 0.25) (layer B.Cu) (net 1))
 (segment (start 144.7738 115.782) (end 144.7738 117.4612) (width 0.25) (layer B.Cu) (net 1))
 (segment (start 144.02 99.2437) (end 144.690001 98.573699) (width 0.25) (layer F.Cu) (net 1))
 (segment (start 125.64 122.1) (end 125.64 123.25) (width 0.25) (layer F.Cu) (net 1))
 (segment (start 126.41 121.33) (end 125.64 122.1) (width 0.25) (layer F.Cu) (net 1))
 (segment (start 134.74 120.23) (end 133.64 121.33) (width 0.25) (layer F.Cu) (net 1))
 (segment (start 134.74 117.9) (end 134.74 120.23) (width 0.25) (layer F.Cu) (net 1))
 (via (at 130.12 121.33) (size 0.8) (drill 0.4) (layers F.Cu B.Cu) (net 1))
 (segment (start 130.12 118.7506) (end 130.12 121.33) (width 0.25) (layer B.Cu) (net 1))
 (segment (start 130.12 121.33) (end 126.41 121.33) (width 0.25) (layer F.Cu) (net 1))
 (segment (start 128.4244 117.055) (end 130.12 118.7506) (width 0.25) (layer B.Cu) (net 1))
 (segment (start 127.0822 117.055) (end 128.4244 117.055) (width 0.25) (layer B.Cu) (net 1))
 (segment (start 133.64 121.33) (end 130.12 121.33) (width 0.25) (layer F.Cu) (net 1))
 (via (at 144.78 114.046) (size 0.8) (drill 0.4) (layers F.Cu B.Cu) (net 1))
 (segment (start 144.7738 114.0522) (end 144.78 114.046) (width 0.25) (layer B.Cu) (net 1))
 (segment (start 144.7738 115.782) (end 144.7738 114.0522) (width 0.25) (layer B.Cu) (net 1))
 (segment (start 144.78 114.046) (end 146.05 114.046) (width 0.25) (layer F.Cu) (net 1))
 (via (at 143.256 108.204) (size 0.8) (drill 0.4) (layers F.Cu B.Cu) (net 1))
 (segment (start 142.865 108.595) (end 143.256 108.204) (width 0.25) (layer B.Cu) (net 1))
 (segment (start 142.865 109.65) (end 142.865 108.595) (width 0.25) (layer B.Cu) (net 1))
 (segment (start 143.256 108.204) (end 146.05 108.204) (width 0.25) (layer F.Cu) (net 1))
 (segment (start 146.05 114.046) (end 146.05 108.204) (width 0.25) (layer F.Cu) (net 1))
 (via (at 131.318 110.236) (size 0.8) (drill 0.4) (layers F.Cu B.Cu) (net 1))
 (segment (start 131.352 110.27) (end 131.318 110.236) (width 0.25) (layer B.Cu) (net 1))
 (segment (start 133.585 110.27) (end 131.352 110.27) (width 0.25) (layer B.Cu) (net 1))
 (segment (start 133.394 117.9) (end 134.74 117.9) (width 0.25) (layer F.Cu) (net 1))
 (segment (start 129.21 113.716) (end 133.394 117.9) (width 0.25) (layer F.Cu) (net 1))
 (segment (start 129.21 113.39) (end 129.21 113.716) (width 0.25) (layer F.Cu) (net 1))
 (segment (start 144.428 103.28) (end 144.02 103.28) (width 0.25) (layer F.Cu) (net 1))
 (segment (start 146.05 104.902) (end 144.428 103.28) (width 0.25) (layer F.Cu) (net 1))
 (segment (start 146.05 108.204) (end 146.05 104.902) (width 0.25) (layer F.Cu) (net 1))
 (segment (start 138.178002 99.107702) (end 138.277999 99.207699) (width 1) (layer F.Cu) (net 1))
 (segment (start 138.178002 96.757698) (end 138.178002 99.107702) (width 1) (layer F.Cu) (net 1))
 (segment (start 144.777998 99.107702) (end 144.678001 99.207699) (width 1) (layer F.Cu) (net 1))
 (segment (start 144.777998 96.757698) (end 144.777998 99.107702) (width 1) (layer F.Cu) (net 1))
 (segment (start 138.178002 96.757698) (end 144.777998 96.757698) (width 1) (layer F.Cu) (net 1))
 (segment (start 122.126 98.346) (end 122.126 103.554) (width 0.25) (layer F.Cu) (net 1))
 (segment (start 123.698 96.774) (end 122.126 98.346) (width 0.25) (layer F.Cu) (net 1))
 (segment (start 134.62 96.774) (end 123.698 96.774) (width 0.25) (layer F.Cu) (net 1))
 (segment (start 137.053699 99.207699) (end 134.62 96.774) (width 0.25) (layer F.Cu) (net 1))
 (segment (start 138.277999 99.207699) (end 137.053699 99.207699) (width 0.25) (layer F.Cu) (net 1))
 (segment (start 138.502999 99.432699) (end 138.277999 99.207699) (width 0.25) (layer F.Cu) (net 1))
 (segment (start 140.178 99.432699) (end 138.502999 99.432699) (width 0.25) (layer F.Cu) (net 1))
 (segment (start 144.02 99.8657) (end 144.678001 99.207699) (width 0.25) (layer F.Cu) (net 1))
 (segment (start 144.02 103.28) (end 144.02 99.8657) (width 0.25) (layer F.Cu) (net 1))
 (segment (start 146.05 118.39) (end 146.05 114.046) (width 0.25) (layer F.Cu) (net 1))
 (segment (start 143.93 120.51) (end 146.05 118.39) (width 0.25) (layer F.Cu) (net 1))
 (segment (start 134.46 120.51) (end 143.93 120.51) (width 0.25) (layer F.Cu) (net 1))
 (segment (start 133.64 121.33) (end 134.46 120.51) (width 0.25) (layer F.Cu) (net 1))
 (segment (start 134.83 117.9) (end 134.74 117.9) (width 0.25) (layer F.Cu) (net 1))
 (segment (start 136.398 116.332) (end 134.83 117.9) (width 0.25) (layer F.Cu) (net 1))
 (segment (start 136.398 111.252) (end 136.398 116.332) (width 0.25) (layer F.Cu) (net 1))
 (segment (start 135.416 110.27) (end 136.398 111.252) (width 0.25) (layer F.Cu) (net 1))
 (segment (start 131.352 110.27) (end 135.416 110.27) (width 0.25) (layer F.Cu) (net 1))
 (segment (start 131.318 110.236) (end 131.352 110.27) (width 0.25) (layer F.Cu) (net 1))
 (segment (start 140.208 104.548) (end 138.94 103.28) (width 0.25) (layer B.Cu) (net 5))
 (segment (start 140.208 109.728) (end 140.208 104.548) (width 0.25) (layer B.Cu) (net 5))
 (segment (start 139.666 110.27) (end 140.208 109.728) (width 0.25) (layer B.Cu) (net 5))
 (segment (start 138.535 110.27) (end 139.666 110.27) (width 0.25) (layer B.Cu) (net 5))
 (segment (start 142.494 101.346) (end 142.79 101.05) (width 0.25) (layer F.Cu) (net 5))
 (segment (start 139.7 101.346) (end 142.494 101.346) (width 0.25) (layer F.Cu) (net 5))
 (segment (start 138.94 102.106) (end 139.7 101.346) (width 0.25) (layer F.Cu) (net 5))
 (segment (start 138.94 103.28) (end 138.94 102.106) (width 0.25) (layer F.Cu) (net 5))
 (segment (start 136.906 110.924) (end 137.56 110.27) (width 0.25) (layer B.Cu) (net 5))
 (segment (start 137.56 110.27) (end 138.535 110.27) (width 0.25) (layer B.Cu) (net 5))
 (segment (start 136.906 118.676) (end 136.906 110.924) (width 0.25) (layer B.Cu) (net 5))
 (segment (start 138.43 120.2) (end 136.906 118.676) (width 0.25) (layer B.Cu) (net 5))
 (segment (start 138.43 125.65) (end 138.43 120.2) (width 0.25) (layer B.Cu) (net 5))
 (segment (start 125.99 127.63) (end 136.45 127.63) (width 0.25) (layer B.Cu) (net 5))
 (segment (start 136.45 127.63) (end 138.43 125.65) (width 0.25) (layer B.Cu) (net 5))
 (segment (start 124.24 125.88) (end 125.99 127.63) (width 0.25) (layer B.Cu) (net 5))
 (segment (start 124.24 119.199) (end 124.24 125.88) (width 0.25) (layer B.Cu) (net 5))
 (segment (start 125.114 118.325) (end 124.24 119.199) (width 0.25) (layer B.Cu) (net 5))
 (segment (start 127.0822 118.325) (end 125.114 118.325) (width 0.25) (layer B.Cu) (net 5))
 (segment (start 142.778 101.038) (end 142.79 101.05) (width 0.25) (layer F.Cu) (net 5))
 (segment (start 142.778 99.432699) (end 142.778 101.038) (width 0.25) (layer F.Cu) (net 5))
 (segment (start 138.94 102.11) (end 138.94 103.28) (width 0.25) (layer B.Cu) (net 5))
 (segment (start 138.2 101.37) (end 138.94 102.11) (width 0.25) (layer B.Cu) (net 5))
 (segment (start 135.864998 101.37) (end 138.2 101.37) (width 0.25) (layer B.Cu) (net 5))
 (segment (start 133.680998 103.554) (end 135.864998 101.37) (width 0.25) (layer B.Cu) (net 5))
 (segment (start 128.826 103.554) (end 133.680998 103.554) (width 0.25) (layer B.Cu) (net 5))
 (segment (start 132.8 114.08) (end 133.585 114.08) (width 0.25) (layer B.Cu) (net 17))
 (segment (start 128.155 109.435) (end 132.8 114.08) (width 0.25) (layer B.Cu) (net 17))
 (segment (start 127.0822 109.435) (end 128.155 109.435) (width 0.25) (layer B.Cu) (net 17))
 (segment (start 134.654 112.81) (end 133.585 112.81) (width 0.25) (layer B.Cu) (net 16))
 (segment (start 134.88501 113.04101) (end 134.654 112.81) (width 0.25) (layer B.Cu) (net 16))
 (segment (start 134.88501 114.426758) (end 134.88501 113.04101) (width 0.25) (layer B.Cu) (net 16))
 (segment (start 134.606758 114.70501) (end 134.88501 114.426758) (width 0.25) (layer B.Cu) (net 16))
 (segment (start 132.563242 114.70501) (end 134.606758 114.70501) (width 0.25) (layer B.Cu) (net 16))
 (segment (start 128.563232 110.705) (end 132.563242 114.70501) (width 0.25) (layer B.Cu) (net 16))
 (segment (start 127.0822 110.705) (end 128.563232 110.705) (width 0.25) (layer B.Cu) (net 16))
 (segment (start 131.352 111.54) (end 133.585 111.54) (width 0.25) (layer B.Cu) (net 15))
 (segment (start 128.272 108.46) (end 131.352 111.54) (width 0.25) (layer B.Cu) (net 15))
 (segment (start 125.68 108.46) (end 128.272 108.46) (width 0.25) (layer B.Cu) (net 15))
 (segment (start 125.15 108.99) (end 125.68 108.46) (width 0.25) (layer B.Cu) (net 15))
 (segment (start 125.74 113.245) (end 125.15 112.655) (width 0.25) (layer B.Cu) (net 15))
 (segment (start 125.15 112.655) (end 125.15 108.99) (width 0.25) (layer B.Cu) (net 15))
 (segment (start 127.0822 113.245) (end 125.74 113.245) (width 0.25) (layer B.Cu) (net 15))
 (segment (start 134.4 104.15) (end 135.29 103.26) (width 0.25) (layer B.Cu) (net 18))
 (segment (start 134.4 107.29) (end 134.4 104.15) (width 0.25) (layer B.Cu) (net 18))
 (segment (start 135.40997 108.29997) (end 134.4 107.29) (width 0.25) (layer B.Cu) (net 18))
 (segment (start 135.40997 114.538208) (end 135.40997 108.29997) (width 0.25) (layer B.Cu) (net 18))
 (segment (start 134.598178 115.35) (end 135.40997 114.538208) (width 0.25) (layer B.Cu) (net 18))
 (segment (start 135.29 103.26) (end 136.26 103.26) (width 0.25) (layer B.Cu) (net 18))
 (segment (start 133.585 115.35) (end 134.598178 115.35) (width 0.25) (layer B.Cu) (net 18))
 (segment (start 139.601008 111.54) (end 138.535 111.54) (width 0.25) (layer B.Cu) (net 13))
 (segment (start 144.415 111.3592) (end 144.7738 111.718) (width 0.25) (layer B.Cu) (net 13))
 (segment (start 144.415 109.65) (end 144.415 111.3592) (width 0.25) (layer B.Cu) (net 13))
 (segment (start 144.7738 112.7262) (end 144.7738 111.718) (width 0.25) (layer B.Cu) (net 13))
 (segment (start 144.11 113.39) (end 144.7738 112.7262) (width 0.25) (layer B.Cu) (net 13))
 (segment (start 141.55 113.39) (end 144.11 113.39) (width 0.25) (layer B.Cu) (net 13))
 (segment (start 139.7 111.54) (end 141.55 113.39) (width 0.25) (layer B.Cu) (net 13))
 (segment (start 138.535 111.54) (end 139.7 111.54) (width 0.25) (layer B.Cu) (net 13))
 (segment (start 139.4159 112.81) (end 138.535 112.81) (width 0.25) (layer B.Cu) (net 14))
 (segment (start 142.755 116.1508) (end 142.3862 115.782) (width 0.25) (layer B.Cu) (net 14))
 (segment (start 142.755 117.93) (end 142.755 116.1508) (width 0.25) (layer B.Cu) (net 14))
 (segment (start 139.86 112.81) (end 142.3862 115.3362) (width 0.25) (layer B.Cu) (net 14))
 (segment (start 142.3862 115.3362) (end 142.3862 115.782) (width 0.25) (layer B.Cu) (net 14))
 (segment (start 138.535 112.81) (end 139.86 112.81) (width 0.25) (layer B.Cu) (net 14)))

